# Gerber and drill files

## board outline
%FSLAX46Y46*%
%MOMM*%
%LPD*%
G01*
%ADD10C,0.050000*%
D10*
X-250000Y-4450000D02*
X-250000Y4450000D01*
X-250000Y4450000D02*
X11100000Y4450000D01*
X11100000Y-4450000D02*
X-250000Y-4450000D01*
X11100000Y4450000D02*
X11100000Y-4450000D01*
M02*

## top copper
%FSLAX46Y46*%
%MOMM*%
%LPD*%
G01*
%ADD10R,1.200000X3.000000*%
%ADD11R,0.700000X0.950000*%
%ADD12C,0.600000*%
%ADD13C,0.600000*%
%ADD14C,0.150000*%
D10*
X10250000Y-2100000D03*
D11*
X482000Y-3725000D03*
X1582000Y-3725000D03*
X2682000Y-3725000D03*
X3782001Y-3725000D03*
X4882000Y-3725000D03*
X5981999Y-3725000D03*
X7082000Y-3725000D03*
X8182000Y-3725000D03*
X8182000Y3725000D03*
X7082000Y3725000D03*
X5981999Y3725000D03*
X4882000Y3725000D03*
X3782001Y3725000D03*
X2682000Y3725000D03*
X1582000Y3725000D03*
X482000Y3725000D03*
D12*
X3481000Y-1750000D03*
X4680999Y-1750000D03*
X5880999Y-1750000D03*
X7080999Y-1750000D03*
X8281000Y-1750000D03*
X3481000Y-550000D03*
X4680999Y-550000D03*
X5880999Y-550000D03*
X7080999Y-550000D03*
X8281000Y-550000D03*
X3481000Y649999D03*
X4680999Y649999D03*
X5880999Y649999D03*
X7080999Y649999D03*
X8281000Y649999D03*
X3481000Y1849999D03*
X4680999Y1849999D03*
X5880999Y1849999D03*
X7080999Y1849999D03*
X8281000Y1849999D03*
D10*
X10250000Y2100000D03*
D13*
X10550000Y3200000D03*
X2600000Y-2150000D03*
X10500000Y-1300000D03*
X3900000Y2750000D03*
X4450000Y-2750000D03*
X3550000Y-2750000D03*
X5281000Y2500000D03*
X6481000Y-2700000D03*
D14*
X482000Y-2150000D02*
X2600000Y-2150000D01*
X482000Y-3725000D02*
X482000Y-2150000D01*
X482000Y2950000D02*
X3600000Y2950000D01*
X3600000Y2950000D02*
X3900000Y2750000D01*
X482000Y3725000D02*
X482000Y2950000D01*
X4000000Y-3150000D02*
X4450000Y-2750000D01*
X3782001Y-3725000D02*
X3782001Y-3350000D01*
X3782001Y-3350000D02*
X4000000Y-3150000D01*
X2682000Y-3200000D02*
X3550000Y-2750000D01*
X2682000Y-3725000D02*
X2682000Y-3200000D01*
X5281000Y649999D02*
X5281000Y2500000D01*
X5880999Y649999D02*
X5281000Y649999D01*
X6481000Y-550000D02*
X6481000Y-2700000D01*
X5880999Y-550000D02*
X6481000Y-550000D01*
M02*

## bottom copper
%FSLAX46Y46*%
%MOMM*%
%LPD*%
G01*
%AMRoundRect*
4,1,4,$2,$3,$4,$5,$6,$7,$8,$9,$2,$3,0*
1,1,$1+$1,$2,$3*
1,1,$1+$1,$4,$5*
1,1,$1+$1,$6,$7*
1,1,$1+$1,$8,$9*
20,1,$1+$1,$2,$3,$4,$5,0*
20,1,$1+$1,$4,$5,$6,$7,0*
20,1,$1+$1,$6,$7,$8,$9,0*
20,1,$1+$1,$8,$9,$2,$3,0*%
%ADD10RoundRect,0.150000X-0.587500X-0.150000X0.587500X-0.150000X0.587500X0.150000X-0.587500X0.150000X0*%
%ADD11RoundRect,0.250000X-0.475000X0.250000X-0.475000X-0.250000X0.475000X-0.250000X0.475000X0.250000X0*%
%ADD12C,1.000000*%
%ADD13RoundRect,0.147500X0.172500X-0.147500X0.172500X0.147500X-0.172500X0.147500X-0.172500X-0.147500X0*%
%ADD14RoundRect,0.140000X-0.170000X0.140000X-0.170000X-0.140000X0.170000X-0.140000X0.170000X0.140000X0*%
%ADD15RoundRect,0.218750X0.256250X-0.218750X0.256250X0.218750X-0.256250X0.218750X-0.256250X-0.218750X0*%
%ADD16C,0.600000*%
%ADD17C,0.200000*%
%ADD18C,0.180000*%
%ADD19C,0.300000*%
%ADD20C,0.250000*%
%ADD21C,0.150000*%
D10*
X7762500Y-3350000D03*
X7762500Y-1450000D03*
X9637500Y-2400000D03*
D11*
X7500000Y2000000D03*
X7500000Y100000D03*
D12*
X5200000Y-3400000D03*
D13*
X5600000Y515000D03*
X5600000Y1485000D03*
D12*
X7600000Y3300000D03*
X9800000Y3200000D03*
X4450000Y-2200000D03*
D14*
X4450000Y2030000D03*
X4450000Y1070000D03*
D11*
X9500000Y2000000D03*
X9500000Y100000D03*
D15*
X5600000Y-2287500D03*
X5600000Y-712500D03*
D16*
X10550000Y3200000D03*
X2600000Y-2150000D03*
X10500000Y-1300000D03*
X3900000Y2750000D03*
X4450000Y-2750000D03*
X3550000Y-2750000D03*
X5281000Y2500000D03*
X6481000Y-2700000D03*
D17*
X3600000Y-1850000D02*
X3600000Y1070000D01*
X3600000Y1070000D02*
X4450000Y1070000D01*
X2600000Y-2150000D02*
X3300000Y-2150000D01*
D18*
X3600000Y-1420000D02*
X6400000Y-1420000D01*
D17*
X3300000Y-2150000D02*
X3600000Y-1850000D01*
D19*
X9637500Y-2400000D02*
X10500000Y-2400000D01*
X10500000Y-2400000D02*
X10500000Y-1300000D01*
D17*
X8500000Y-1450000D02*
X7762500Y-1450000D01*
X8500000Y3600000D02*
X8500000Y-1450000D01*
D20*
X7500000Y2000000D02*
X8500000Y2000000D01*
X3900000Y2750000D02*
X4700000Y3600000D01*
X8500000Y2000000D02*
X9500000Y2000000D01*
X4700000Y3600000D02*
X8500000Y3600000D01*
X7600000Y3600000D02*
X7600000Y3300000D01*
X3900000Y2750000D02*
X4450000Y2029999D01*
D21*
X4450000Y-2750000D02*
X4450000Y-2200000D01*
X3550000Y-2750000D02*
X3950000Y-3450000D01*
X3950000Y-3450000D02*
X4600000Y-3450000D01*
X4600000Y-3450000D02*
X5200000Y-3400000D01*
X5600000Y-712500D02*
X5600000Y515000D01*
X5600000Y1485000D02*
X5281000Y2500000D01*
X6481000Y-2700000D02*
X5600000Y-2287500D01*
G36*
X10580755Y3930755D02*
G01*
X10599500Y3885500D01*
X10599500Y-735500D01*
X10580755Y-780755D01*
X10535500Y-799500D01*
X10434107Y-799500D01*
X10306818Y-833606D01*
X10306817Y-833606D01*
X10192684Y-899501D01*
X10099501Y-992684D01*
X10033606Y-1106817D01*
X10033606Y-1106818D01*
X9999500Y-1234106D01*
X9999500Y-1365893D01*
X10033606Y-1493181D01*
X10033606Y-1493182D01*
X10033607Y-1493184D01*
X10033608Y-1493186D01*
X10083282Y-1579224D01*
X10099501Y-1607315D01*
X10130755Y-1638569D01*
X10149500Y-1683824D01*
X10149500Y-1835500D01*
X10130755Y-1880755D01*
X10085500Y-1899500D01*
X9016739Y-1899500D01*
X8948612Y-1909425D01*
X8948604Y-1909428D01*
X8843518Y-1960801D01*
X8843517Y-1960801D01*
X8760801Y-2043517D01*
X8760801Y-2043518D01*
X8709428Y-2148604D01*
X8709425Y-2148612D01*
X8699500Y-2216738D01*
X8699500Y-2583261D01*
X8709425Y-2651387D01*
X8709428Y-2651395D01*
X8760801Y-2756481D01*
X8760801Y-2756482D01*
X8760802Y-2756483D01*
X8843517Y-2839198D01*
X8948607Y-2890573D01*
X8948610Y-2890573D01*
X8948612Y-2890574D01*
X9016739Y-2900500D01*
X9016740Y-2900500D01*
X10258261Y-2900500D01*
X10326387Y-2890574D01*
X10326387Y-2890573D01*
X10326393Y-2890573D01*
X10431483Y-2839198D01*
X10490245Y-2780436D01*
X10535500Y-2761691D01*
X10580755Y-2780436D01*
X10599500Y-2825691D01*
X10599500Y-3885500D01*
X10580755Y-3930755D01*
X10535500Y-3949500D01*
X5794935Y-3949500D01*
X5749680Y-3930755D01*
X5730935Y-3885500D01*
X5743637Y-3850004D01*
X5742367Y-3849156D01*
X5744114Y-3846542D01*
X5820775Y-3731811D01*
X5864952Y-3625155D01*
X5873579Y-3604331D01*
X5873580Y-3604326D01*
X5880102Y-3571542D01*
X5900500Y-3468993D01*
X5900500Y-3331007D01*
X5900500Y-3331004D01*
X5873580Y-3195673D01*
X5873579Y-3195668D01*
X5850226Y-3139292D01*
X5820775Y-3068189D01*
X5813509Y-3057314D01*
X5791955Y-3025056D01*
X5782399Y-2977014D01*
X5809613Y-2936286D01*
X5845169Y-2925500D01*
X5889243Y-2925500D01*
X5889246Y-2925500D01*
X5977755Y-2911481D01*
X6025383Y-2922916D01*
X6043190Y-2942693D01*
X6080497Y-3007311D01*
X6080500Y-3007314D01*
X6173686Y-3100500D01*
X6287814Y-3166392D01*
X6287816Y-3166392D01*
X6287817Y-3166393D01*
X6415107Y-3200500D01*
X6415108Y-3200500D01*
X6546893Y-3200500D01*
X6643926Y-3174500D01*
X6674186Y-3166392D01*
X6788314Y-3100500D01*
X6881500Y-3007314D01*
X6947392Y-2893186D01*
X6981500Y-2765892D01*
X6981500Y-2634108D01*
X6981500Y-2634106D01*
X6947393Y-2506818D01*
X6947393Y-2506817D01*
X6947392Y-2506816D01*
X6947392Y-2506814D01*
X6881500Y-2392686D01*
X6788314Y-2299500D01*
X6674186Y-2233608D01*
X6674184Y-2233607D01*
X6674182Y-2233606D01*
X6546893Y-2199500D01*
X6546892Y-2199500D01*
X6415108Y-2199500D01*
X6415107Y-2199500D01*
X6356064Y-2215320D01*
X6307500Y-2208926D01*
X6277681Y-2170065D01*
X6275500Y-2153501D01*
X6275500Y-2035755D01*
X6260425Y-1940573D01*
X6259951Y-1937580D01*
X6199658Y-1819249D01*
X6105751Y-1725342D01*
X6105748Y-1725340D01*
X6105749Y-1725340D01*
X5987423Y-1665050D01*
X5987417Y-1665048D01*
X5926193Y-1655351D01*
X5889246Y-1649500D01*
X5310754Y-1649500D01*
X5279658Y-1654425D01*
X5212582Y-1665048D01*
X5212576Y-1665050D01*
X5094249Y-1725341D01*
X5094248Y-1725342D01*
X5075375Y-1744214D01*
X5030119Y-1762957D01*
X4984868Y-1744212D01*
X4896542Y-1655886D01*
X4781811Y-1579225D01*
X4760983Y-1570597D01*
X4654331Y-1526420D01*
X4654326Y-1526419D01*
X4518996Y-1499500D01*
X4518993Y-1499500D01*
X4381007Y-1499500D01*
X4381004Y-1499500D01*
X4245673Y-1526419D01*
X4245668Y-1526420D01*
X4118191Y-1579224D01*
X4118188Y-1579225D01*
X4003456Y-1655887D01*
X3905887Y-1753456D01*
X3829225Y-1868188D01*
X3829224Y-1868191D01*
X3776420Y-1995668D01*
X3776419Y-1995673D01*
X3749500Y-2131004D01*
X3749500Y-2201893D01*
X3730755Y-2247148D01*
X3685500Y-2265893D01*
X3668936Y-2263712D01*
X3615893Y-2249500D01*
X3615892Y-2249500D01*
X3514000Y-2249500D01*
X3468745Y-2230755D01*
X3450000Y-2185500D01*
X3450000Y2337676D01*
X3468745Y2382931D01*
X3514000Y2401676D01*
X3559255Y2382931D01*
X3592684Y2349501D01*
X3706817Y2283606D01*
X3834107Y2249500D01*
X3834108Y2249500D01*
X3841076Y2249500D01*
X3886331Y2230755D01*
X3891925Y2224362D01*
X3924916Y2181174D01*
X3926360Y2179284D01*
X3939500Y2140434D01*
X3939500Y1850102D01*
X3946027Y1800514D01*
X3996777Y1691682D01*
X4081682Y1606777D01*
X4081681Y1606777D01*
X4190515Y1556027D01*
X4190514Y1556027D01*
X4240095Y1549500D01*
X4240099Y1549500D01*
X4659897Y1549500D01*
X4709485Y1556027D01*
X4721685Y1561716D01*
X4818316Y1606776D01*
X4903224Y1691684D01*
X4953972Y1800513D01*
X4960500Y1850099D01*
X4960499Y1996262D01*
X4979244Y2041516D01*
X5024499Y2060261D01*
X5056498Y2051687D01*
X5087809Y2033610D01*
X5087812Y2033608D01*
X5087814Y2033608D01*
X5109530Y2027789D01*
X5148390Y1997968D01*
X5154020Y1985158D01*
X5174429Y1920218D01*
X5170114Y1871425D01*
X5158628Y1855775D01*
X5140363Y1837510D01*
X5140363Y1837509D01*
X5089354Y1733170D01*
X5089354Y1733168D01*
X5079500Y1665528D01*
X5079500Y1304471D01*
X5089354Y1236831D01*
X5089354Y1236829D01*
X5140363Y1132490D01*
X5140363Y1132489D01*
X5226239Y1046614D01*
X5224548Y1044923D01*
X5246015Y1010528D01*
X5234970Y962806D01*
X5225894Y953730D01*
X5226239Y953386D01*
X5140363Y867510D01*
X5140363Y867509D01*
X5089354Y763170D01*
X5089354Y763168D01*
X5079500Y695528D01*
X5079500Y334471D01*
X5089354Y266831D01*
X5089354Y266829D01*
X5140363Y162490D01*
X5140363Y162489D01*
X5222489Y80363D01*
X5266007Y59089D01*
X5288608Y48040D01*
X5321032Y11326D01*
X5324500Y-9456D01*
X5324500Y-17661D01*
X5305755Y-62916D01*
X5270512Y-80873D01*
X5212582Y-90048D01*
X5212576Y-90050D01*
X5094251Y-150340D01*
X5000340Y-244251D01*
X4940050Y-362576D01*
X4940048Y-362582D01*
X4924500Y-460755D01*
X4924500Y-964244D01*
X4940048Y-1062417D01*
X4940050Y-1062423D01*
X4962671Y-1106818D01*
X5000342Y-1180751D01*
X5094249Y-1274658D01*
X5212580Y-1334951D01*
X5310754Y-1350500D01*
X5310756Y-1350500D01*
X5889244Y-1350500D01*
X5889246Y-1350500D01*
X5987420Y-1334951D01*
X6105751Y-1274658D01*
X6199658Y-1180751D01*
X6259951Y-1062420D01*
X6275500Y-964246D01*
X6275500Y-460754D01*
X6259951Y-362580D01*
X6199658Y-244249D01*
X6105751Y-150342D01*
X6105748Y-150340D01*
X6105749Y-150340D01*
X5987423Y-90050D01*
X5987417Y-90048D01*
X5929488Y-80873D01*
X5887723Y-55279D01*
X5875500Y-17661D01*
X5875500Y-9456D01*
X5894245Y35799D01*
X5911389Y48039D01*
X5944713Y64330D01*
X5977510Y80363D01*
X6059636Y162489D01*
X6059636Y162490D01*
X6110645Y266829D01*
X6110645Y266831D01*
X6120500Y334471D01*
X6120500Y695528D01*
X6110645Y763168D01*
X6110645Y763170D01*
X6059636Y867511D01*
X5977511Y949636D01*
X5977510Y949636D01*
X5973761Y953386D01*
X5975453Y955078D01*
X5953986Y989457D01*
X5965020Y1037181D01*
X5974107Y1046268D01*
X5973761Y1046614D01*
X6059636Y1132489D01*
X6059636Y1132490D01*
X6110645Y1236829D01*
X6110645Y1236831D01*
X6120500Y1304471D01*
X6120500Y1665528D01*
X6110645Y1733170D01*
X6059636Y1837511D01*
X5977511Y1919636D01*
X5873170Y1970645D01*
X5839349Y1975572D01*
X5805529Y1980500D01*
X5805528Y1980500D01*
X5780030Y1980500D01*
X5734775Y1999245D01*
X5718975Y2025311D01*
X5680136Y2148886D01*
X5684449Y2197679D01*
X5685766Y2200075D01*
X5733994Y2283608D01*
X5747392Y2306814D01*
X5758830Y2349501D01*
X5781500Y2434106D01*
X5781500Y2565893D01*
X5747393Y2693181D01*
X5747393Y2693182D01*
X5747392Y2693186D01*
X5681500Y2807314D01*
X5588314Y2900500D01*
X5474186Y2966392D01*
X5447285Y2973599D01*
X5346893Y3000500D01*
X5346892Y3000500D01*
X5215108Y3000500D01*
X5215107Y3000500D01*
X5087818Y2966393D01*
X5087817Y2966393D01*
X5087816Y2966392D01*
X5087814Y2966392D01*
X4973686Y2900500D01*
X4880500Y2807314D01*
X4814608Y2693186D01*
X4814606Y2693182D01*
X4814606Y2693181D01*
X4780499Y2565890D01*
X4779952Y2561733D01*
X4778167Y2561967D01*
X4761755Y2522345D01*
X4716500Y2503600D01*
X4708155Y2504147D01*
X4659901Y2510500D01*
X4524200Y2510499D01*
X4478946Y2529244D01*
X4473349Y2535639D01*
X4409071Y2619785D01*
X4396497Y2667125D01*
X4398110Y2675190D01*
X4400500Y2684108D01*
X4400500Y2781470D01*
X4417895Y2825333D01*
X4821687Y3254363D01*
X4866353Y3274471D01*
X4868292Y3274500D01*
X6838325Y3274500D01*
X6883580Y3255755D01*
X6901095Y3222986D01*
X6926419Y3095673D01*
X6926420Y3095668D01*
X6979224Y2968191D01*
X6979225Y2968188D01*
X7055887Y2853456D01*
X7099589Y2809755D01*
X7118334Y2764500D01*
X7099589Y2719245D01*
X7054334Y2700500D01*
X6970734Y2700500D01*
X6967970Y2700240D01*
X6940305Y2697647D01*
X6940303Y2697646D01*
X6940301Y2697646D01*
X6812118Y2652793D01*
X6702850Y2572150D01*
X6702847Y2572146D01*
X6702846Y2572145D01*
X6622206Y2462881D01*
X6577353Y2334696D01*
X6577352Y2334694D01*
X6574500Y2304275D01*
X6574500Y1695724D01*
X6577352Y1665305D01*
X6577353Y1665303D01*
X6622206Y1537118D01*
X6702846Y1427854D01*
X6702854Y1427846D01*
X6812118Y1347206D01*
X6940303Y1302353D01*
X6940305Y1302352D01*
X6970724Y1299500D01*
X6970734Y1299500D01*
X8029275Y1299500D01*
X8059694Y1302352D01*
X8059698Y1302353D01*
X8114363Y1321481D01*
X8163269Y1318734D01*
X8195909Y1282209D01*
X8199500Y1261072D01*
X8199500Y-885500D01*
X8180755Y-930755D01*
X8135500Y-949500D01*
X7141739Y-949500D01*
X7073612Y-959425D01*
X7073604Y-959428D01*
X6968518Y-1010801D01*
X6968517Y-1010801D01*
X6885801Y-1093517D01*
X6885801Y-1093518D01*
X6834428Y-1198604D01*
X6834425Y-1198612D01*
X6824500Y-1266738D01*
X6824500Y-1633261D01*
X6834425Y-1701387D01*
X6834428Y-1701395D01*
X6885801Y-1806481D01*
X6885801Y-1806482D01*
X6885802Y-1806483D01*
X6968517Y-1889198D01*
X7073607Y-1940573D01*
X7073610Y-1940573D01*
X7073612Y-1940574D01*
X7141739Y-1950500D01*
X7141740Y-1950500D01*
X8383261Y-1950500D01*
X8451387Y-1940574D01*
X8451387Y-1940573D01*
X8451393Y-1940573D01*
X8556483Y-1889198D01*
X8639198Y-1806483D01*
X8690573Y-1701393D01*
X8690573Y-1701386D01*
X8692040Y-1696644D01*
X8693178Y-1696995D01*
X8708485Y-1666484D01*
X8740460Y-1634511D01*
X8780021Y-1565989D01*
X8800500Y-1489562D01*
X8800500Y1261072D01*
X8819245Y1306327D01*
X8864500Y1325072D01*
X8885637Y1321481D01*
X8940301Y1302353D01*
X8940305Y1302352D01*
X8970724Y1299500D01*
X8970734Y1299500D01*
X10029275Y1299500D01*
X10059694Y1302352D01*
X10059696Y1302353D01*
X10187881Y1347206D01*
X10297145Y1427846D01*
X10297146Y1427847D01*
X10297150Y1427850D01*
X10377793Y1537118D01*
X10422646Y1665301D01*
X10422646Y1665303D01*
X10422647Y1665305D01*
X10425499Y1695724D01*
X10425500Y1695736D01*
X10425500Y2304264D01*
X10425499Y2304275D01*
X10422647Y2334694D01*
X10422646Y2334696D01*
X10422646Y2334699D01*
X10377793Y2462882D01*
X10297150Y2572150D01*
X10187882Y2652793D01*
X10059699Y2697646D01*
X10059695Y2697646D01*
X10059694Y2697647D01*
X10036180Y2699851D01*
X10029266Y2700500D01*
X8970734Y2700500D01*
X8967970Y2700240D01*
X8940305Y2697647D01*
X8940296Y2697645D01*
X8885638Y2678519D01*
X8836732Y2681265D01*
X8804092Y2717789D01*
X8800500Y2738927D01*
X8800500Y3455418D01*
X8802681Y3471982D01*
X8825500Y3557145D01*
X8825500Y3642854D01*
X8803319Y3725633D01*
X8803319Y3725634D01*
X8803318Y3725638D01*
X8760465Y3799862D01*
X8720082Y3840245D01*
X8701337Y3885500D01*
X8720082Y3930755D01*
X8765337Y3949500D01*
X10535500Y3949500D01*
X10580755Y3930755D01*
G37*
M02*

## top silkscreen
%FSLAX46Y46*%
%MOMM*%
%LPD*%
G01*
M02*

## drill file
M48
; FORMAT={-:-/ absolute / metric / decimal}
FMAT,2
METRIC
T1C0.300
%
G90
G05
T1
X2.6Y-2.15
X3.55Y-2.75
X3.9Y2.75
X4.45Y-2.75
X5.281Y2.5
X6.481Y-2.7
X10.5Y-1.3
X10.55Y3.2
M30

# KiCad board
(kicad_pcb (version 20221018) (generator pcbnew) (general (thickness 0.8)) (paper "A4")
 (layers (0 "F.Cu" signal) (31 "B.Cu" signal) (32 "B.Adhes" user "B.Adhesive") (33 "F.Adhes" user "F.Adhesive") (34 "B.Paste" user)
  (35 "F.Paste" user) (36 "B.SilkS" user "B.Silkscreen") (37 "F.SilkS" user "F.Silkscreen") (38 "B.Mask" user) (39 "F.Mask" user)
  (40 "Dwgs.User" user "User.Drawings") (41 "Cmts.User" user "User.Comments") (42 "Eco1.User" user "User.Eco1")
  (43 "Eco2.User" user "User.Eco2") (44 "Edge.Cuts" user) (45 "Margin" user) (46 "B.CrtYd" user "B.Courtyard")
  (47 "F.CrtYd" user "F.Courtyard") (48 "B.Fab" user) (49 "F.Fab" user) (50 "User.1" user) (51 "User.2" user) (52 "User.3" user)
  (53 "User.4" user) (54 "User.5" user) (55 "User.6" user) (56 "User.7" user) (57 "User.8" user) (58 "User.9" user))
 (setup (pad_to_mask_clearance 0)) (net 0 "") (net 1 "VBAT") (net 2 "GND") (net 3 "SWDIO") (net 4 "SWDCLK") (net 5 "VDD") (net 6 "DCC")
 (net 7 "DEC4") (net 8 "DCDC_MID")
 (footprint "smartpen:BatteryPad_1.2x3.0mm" (layer "F.Cu") (at 10.25 2.1)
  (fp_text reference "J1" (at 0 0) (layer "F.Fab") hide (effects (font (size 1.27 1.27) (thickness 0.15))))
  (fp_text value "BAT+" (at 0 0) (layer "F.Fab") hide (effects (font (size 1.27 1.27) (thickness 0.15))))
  (pad "1" smd rect (at 0 0) (size 1.2 3) (layers "F.Cu" "F.Mask") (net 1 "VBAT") (thermal_bridge_angle 45)))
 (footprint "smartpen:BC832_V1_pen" (layer "F.Cu") (at 4.4 0 90)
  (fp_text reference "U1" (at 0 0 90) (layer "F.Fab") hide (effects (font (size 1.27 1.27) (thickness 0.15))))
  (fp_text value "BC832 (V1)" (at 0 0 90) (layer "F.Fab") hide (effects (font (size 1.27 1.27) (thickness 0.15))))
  (pad "1" smd rect (at -3.725 -3.918 90) (size 0.95 0.7) (layers "F.Cu" "F.Paste" "F.Mask") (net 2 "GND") (thermal_bridge_angle 45))
  (pad "2" smd rect (at -3.725 -2.818 90) (size 0.95 0.7) (layers "F.Cu" "F.Paste" "F.Mask") (thermal_bridge_angle 45))
  (pad "3" smd rect (at -3.725 -1.718 90) (size 0.95 0.7) (layers "F.Cu" "F.Paste" "F.Mask") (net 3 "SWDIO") (thermal_bridge_angle 45))
  (pad "4" smd rect (at -3.725 -0.617999 90) (size 0.95 0.7) (layers "F.Cu" "F.Paste" "F.Mask") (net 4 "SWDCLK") (thermal_bridge_angle 45))
  (pad "5" smd rect (at -3.725 0.482 90) (size 0.95 0.7) (layers "F.Cu" "F.Paste" "F.Mask") (thermal_bridge_angle 45))
  (pad "6" smd rect (at -3.725 1.581999 90) (size 0.95 0.7) (layers "F.Cu" "F.Paste" "F.Mask") (thermal_bridge_angle 45))
  (pad "7" smd rect (at -3.725 2.682 90) (size 0.95 0.7) (layers "F.Cu" "F.Paste" "F.Mask") (thermal_bridge_angle 45))
  (pad "8" smd rect (at -3.725 3.782 90) (size 0.95 0.7) (layers "F.Cu" "F.Paste" "F.Mask") (thermal_bridge_angle 45))
  (pad "9" smd rect (at 3.725 3.782 90) (size 0.95 0.7) (layers "F.Cu" "F.Paste" "F.Mask") (thermal_bridge_angle 45))
  (pad "10" smd rect (at 3.725 2.682 90) (size 0.95 0.7) (layers "F.Cu" "F.Paste" "F.Mask") (thermal_bridge_angle 45))
  (pad "11" smd rect (at 3.725 1.581999 90) (size 0.95 0.7) (layers "F.Cu" "F.Paste" "F.Mask") (thermal_bridge_angle 45))
  (pad "12" smd rect (at 3.725 0.482 90) (size 0.95 0.7) (layers "F.Cu" "F.Paste" "F.Mask") (thermal_bridge_angle 45))
  (pad "13" smd rect (at 3.725 -0.617999 90) (size 0.95 0.7) (layers "F.Cu" "F.Paste" "F.Mask") (thermal_bridge_angle 45))
  (pad "14" smd rect (at 3.725 -1.718 90) (size 0.95 0.7) (layers "F.Cu" "F.Paste" "F.Mask") (thermal_bridge_angle 45))
  (pad "15" smd rect (at 3.725 -2.818 90) (size 0.95 0.7) (layers "F.Cu" "F.Paste" "F.Mask") (thermal_bridge_angle 45))
  (pad "16" smd rect (at 3.725 -3.918 90) (size 0.95 0.7) (layers "F.Cu" "F.Paste" "F.Mask") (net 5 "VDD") (thermal_bridge_angle 45))
  (pad "A1" smd circle (at -1.75 -0.919 90) (size 0.6 0.6) (layers "F.Cu" "F.Paste" "F.Mask"))
  (pad "A2" smd circle (at -1.75 0.280999 90) (size 0.6 0.6) (layers "F.Cu" "F.Paste" "F.Mask"))
  (pad "A3" smd circle (at -1.75 1.480999 90) (size 0.6 0.6) (layers "F.Cu" "F.Paste" "F.Mask"))
  (pad "A4" smd circle (at -1.75 2.680999 90) (size 0.6 0.6) (layers "F.Cu" "F.Paste" "F.Mask"))
  (pad "A5" smd circle (at -1.75 3.881 90) (size 0.6 0.6) (layers "F.Cu" "F.Paste" "F.Mask"))
  (pad "B1" smd circle (at -0.55 -0.919 90) (size 0.6 0.6) (layers "F.Cu" "F.Paste" "F.Mask"))
  (pad "B2" smd circle (at -0.55 0.280999 90) (size 0.6 0.6) (layers "F.Cu" "F.Paste" "F.Mask"))
  (pad "B3" smd circle (at -0.55 1.480999 90) (size 0.6 0.6) (layers "F.Cu" "F.Paste" "F.Mask") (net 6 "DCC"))
  (pad "B4" smd circle (at -0.55 2.680999 90) (size 0.6 0.6) (layers "F.Cu" "F.Paste" "F.Mask"))
  (pad "B5" smd circle (at -0.55 3.881 90) (size 0.6 0.6) (layers "F.Cu" "F.Paste" "F.Mask"))
  (pad "C1" smd circle (at 0.649999 -0.919 90) (size 0.6 0.6) (layers "F.Cu" "F.Paste" "F.Mask"))
  (pad "C2" smd circle (at 0.649999 0.280999 90) (size 0.6 0.6) (layers "F.Cu" "F.Paste" "F.Mask"))
  (pad "C3" smd circle (at 0.649999 1.480999 90) (size 0.6 0.6) (layers "F.Cu" "F.Paste" "F.Mask") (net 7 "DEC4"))
  (pad "C4" smd circle (at 0.649999 2.680999 90) (size 0.6 0.6) (layers "F.Cu" "F.Paste" "F.Mask"))
  (pad "C5" smd circle (at 0.649999 3.881 90) (size 0.6 0.6) (layers "F.Cu" "F.Paste" "F.Mask"))
  (pad "D1" smd circle (at 1.849999 -0.919 90) (size 0.6 0.6) (layers "F.Cu" "F.Paste" "F.Mask"))
  (pad "D2" smd circle (at 1.849999 0.280999 90) (size 0.6 0.6) (layers "F.Cu" "F.Paste" "F.Mask"))
  (pad "D3" smd circle (at 1.849999 1.480999 90) (size 0.6 0.6) (layers "F.Cu" "F.Paste" "F.Mask"))
  (pad "D4" smd circle (at 1.849999 2.680999 90) (size 0.6 0.6) (layers "F.Cu" "F.Paste" "F.Mask"))
  (pad "D5" smd circle (at 1.849999 3.881 90) (size 0.6 0.6) (layers "F.Cu" "F.Paste" "F.Mask")))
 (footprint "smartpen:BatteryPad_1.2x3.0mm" (layer "F.Cu") (at 10.25 -2.1)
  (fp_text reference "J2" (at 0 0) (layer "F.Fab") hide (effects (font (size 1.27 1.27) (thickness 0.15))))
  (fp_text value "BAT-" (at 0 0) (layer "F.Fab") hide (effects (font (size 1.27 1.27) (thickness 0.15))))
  (pad "1" smd rect (at 0 0) (size 1.2 3) (layers "F.Cu" "F.Mask") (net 2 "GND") (thermal_bridge_angle 45)))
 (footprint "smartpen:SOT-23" (layer "B.Cu") (at 8.7 2.4)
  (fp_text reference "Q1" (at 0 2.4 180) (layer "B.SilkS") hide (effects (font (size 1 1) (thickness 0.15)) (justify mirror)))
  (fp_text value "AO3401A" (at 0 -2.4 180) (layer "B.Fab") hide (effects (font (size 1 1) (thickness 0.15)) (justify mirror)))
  (pad "1" smd roundrect (at -0.9375 0.95) (size 1.475 0.6) (layers "B.Cu" "B.Paste" "B.Mask") (roundrect_rratio 0.25) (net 2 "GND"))
  (pad "2" smd roundrect (at -0.9375 -0.95) (size 1.475 0.6) (layers "B.Cu" "B.Paste" "B.Mask") (roundrect_rratio 0.25) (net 5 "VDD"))
  (pad "3" smd roundrect (at 0.9375 0) (size 1.475 0.6) (layers "B.Cu" "B.Paste" "B.Mask") (roundrect_rratio 0.25) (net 1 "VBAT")))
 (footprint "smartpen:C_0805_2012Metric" (layer "B.Cu") (at 7.5 -1.05 -90)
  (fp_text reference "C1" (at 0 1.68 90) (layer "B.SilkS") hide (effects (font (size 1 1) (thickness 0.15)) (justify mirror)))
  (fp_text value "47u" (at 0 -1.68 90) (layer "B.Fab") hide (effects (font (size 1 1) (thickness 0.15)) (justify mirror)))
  (pad "1" smd roundrect (at -0.95 0 270) (size 1 1.45) (layers "B.Cu" "B.Paste" "B.Mask") (roundrect_rratio 0.25) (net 5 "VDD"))
  (pad "2" smd roundrect (at 0.95 0 270) (size 1 1.45) (layers "B.Cu" "B.Paste" "B.Mask") (roundrect_rratio 0.25) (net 2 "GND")))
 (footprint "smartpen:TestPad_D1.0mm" (layer "B.Cu") (at 5.2 3.4)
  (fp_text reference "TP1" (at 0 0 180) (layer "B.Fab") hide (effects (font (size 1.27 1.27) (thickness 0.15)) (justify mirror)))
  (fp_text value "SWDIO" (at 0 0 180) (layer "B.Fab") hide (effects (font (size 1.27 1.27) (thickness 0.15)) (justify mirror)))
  (pad "1" smd circle (at 0 0) (size 1 1) (layers "B.Cu" "B.Mask") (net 3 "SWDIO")))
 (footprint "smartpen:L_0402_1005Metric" (layer "B.Cu") (at 5.6 -1 90)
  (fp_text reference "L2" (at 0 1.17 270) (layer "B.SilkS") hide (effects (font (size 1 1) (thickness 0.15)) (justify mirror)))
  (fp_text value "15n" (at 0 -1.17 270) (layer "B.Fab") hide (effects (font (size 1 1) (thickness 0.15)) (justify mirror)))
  (pad "1" smd roundrect (at -0.485 0 90) (size 0.59 0.64) (layers "B.Cu" "B.Paste" "B.Mask") (roundrect_rratio 0.25) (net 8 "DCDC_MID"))
  (pad "2" smd roundrect (at 0.485 0 90) (size 0.59 0.64) (layers "B.Cu" "B.Paste" "B.Mask") (roundrect_rratio 0.25) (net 7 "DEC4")))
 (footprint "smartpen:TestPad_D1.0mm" (layer "B.Cu") (at 7.6 -3.3)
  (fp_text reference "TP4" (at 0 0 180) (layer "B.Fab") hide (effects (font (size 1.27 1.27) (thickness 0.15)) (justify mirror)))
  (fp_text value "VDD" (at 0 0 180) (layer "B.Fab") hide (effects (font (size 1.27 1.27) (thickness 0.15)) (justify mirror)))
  (pad "1" smd circle (at 0 0) (size 1 1) (layers "B.Cu" "B.Mask") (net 5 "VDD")))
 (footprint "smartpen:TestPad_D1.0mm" (layer "B.Cu") (at 9.8 -3.2)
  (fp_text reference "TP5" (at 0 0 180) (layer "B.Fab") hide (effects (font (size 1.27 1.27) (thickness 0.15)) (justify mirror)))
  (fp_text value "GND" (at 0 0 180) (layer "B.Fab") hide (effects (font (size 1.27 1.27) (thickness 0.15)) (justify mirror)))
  (pad "1" smd circle (at 0 0) (size 1 1) (layers "B.Cu" "B.Mask") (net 2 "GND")))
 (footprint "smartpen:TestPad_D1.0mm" (layer "B.Cu") (at 4.45 2.2)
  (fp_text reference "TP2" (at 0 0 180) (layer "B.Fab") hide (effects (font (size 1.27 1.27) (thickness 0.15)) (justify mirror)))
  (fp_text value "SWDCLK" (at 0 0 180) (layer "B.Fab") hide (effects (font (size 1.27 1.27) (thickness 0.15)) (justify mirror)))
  (pad "1" smd circle (at 0 0) (size 1 1) (layers "B.Cu" "B.Mask") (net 4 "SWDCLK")))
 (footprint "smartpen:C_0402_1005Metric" (layer "B.Cu") (at 4.45 -1.55 -90)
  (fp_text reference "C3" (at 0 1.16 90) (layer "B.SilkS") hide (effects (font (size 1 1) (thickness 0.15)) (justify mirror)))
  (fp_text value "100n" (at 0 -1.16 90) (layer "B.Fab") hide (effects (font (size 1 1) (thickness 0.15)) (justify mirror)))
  (pad "1" smd roundrect (at -0.48 0 270) (size 0.56 0.62) (layers "B.Cu" "B.Paste" "B.Mask") (roundrect_rratio 0.25) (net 5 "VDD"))
  (pad "2" smd roundrect (at 0.48 0 270) (size 0.56 0.62) (layers "B.Cu" "B.Paste" "B.Mask") (roundrect_rratio 0.25) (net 2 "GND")))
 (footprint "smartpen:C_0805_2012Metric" (layer "B.Cu") (at 9.5 -1.05 -90)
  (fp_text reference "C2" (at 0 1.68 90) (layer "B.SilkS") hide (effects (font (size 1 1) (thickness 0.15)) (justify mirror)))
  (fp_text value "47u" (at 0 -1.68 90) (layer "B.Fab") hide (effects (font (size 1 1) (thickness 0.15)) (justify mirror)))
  (pad "1" smd roundrect (at -0.95 0 270) (size 1 1.45) (layers "B.Cu" "B.Paste" "B.Mask") (roundrect_rratio 0.25) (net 5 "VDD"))
  (pad "2" smd roundrect (at 0.95 0 270) (size 1 1.45) (layers "B.Cu" "B.Paste" "B.Mask") (roundrect_rratio 0.25) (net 2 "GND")))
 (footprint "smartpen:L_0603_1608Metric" (layer "B.Cu") (at 5.6 1.5 90)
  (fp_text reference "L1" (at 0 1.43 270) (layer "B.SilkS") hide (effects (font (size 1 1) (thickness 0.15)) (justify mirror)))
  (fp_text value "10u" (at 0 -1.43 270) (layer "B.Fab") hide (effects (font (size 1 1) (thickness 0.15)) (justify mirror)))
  (pad "1" smd roundrect (at -0.7875 0 90) (size 0.875 0.95) (layers "B.Cu" "B.Paste" "B.Mask") (roundrect_rratio 0.25) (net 6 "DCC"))
  (pad "2" smd roundrect (at 0.7875 0 90) (size 0.875 0.95) (layers "B.Cu" "B.Paste" "B.Mask") (roundrect_rratio 0.25) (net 8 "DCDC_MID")))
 (gr_line (start -0.25 4.45) (end -0.25 -4.45) (stroke (width 0.05) (type default)) (layer "Edge.Cuts"))
 (gr_line (start -0.25 -4.45) (end 11.1 -4.45) (stroke (width 0.05) (type default)) (layer "Edge.Cuts"))
 (gr_line (start 11.1 4.45) (end -0.25 4.45) (stroke (width 0.05) (type default)) (layer "Edge.Cuts"))
 (gr_line (start 11.1 -4.45) (end 11.1 4.45) (stroke (width 0.05) (type default)) (layer "Edge.Cuts"))
 (segment (start 0.482 2.15) (end 2.6 2.15) (width 0.15) (layer "F.Cu") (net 2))
 (segment (start 0.482 3.725) (end 0.482 2.15) (width 0.15) (layer "F.Cu") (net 2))
 (via (at 10.55 -3.2) (size 0.6) (drill 0.3) (layers "F.Cu" "B.Cu") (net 2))
 (via (at 2.6 2.15) (size 0.6) (drill 0.3) (layers "F.Cu" "B.Cu") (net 2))
 (segment (start 3.6 1.85) (end 3.6 -1.07) (width 0.2) (layer "B.Cu") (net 2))
 (segment (start 3.6 -1.07) (end 4.45 -1.07) (width 0.2) (layer "B.Cu") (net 2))
 (segment (start 2.6 2.15) (end 3.3 2.15) (width 0.2) (layer "B.Cu") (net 2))
 (segment (start 3.6 1.42) (end 6.4 1.42) (width 0.18) (layer "B.Cu") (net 2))
 (segment (start 3.3 2.15) (end 3.6 1.85) (width 0.2) (layer "B.Cu") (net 2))
 (via (at 10.5 1.3) (size 0.6) (drill 0.3) (layers "F.Cu" "B.Cu") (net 1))
 (segment (start 9.6375 2.4) (end 10.5 2.4) (width 0.3) (layer "B.Cu") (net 1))
 (segment (start 10.5 2.4) (end 10.5 1.3) (width 0.3) (layer "B.Cu") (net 1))
 (segment (start 0.482 -2.95) (end 3.6 -2.95) (width 0.15) (layer "F.Cu") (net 5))
 (segment (start 3.6 -2.95) (end 3.9 -2.75) (width 0.15) (layer "F.Cu") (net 5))
 (segment (start 0.482 -3.725) (end 0.482 -2.95) (width 0.15) (layer "F.Cu") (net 5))
 (via (at 3.9 -2.75) (size 0.6) (drill 0.3) (layers "F.Cu" "B.Cu") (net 5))
 (segment (start 8.5 1.45) (end 7.7625 1.45) (width 0.2) (layer "B.Cu") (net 5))
 (segment (start 8.5 -3.6) (end 8.5 1.45) (width 0.2) (layer "B.Cu") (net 5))
 (segment (start 7.5 -2) (end 8.5 -2) (width 0.25) (layer "B.Cu") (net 5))
 (segment (start 3.9 -2.75) (end 4.7 -3.6) (width 0.25) (layer "B.Cu") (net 5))
 (segment (start 8.5 -2) (end 9.5 -2) (width 0.25) (layer "B.Cu") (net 5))
 (segment (start 4.7 -3.6) (end 8.5 -3.6) (width 0.25) (layer "B.Cu") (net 5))
 (segment (start 7.6 -3.6) (end 7.6 -3.3) (width 0.25) (layer "B.Cu") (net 5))
 (segment (start 3.9 -2.75) (end 4.45 -2.029999) (width 0.25) (layer "B.Cu") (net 5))
 (segment (start 4 3.15) (end 4.45 2.75) (width 0.15) (layer "F.Cu") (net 4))
 (segment (start 3.782001 3.725) (end 3.782001 3.35) (width 0.15) (layer "F.Cu") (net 4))
 (segment (start 3.782001 3.35) (end 4 3.15) (width 0.15) (layer "F.Cu") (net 4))
 (via (at 4.45 2.75) (size 0.6) (drill 0.3) (layers "F.Cu" "B.Cu") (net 4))
 (segment (start 4.45 2.75) (end 4.45 2.2) (width 0.15) (layer "B.Cu") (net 4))
 (segment (start 2.682 3.2) (end 3.55 2.75) (width 0.15) (layer "F.Cu") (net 3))
 (segment (start 2.682 3.725) (end 2.682 3.2) (width 0.15) (layer "F.Cu") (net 3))
 (via (at 3.55 2.75) (size 0.6) (drill 0.3) (layers "F.Cu" "B.Cu") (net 3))
 (segment (start 3.55 2.75) (end 3.95 3.45) (width 0.15) (layer "B.Cu") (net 3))
 (segment (start 3.95 3.45) (end 4.6 3.45) (width 0.15) (layer "B.Cu") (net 3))
 (segment (start 4.6 3.45) (end 5.2 3.4) (width 0.15) (layer "B.Cu") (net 3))
 (segment (start 5.6 0.7125) (end 5.6 -0.515) (width 0.15) (layer "B.Cu") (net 8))
 (segment (start 5.281 -0.649999) (end 5.281 -2.5) (width 0.15) (layer "F.Cu") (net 7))
 (segment (start 5.880999 -0.649999) (end 5.281 -0.649999) (width 0.15) (layer "F.Cu") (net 7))
 (via (at 5.281 -2.5) (size 0.6) (drill 0.3) (layers "F.Cu" "B.Cu") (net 7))
 (segment (start 5.6 -1.485) (end 5.281 -2.5) (width 0.15) (layer "B.Cu") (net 7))
 (segment (start 6.481 0.55) (end 6.481 2.7) (width 0.15) (layer "F.Cu") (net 6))
 (segment (start 5.880999 0.55) (end 6.481 0.55) (width 0.15) (layer "F.Cu") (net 6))
 (via (at 6.481 2.7) (size 0.6) (drill 0.3) (layers "F.Cu" "B.Cu") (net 6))
 (segment (start 6.481 2.7) (end 5.6 2.2875) (width 0.15) (layer "B.Cu") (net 6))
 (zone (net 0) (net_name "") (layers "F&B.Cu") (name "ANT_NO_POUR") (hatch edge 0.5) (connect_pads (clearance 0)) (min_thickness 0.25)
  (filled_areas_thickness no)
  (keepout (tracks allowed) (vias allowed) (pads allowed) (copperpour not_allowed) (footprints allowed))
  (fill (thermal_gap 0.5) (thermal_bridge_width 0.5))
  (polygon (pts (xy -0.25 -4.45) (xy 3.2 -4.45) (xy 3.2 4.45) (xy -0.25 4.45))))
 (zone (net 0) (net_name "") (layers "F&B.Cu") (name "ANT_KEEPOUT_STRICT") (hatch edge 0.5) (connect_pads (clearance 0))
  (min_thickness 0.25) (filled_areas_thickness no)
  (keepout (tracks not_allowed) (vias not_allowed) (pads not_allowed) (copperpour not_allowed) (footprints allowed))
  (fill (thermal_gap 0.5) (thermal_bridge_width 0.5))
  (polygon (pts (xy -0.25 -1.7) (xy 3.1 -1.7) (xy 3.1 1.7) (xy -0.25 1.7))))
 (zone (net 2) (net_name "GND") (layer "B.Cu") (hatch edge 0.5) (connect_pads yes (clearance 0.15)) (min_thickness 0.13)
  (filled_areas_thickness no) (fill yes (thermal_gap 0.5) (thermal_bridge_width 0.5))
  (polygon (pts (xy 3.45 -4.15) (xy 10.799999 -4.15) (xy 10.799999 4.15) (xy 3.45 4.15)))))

